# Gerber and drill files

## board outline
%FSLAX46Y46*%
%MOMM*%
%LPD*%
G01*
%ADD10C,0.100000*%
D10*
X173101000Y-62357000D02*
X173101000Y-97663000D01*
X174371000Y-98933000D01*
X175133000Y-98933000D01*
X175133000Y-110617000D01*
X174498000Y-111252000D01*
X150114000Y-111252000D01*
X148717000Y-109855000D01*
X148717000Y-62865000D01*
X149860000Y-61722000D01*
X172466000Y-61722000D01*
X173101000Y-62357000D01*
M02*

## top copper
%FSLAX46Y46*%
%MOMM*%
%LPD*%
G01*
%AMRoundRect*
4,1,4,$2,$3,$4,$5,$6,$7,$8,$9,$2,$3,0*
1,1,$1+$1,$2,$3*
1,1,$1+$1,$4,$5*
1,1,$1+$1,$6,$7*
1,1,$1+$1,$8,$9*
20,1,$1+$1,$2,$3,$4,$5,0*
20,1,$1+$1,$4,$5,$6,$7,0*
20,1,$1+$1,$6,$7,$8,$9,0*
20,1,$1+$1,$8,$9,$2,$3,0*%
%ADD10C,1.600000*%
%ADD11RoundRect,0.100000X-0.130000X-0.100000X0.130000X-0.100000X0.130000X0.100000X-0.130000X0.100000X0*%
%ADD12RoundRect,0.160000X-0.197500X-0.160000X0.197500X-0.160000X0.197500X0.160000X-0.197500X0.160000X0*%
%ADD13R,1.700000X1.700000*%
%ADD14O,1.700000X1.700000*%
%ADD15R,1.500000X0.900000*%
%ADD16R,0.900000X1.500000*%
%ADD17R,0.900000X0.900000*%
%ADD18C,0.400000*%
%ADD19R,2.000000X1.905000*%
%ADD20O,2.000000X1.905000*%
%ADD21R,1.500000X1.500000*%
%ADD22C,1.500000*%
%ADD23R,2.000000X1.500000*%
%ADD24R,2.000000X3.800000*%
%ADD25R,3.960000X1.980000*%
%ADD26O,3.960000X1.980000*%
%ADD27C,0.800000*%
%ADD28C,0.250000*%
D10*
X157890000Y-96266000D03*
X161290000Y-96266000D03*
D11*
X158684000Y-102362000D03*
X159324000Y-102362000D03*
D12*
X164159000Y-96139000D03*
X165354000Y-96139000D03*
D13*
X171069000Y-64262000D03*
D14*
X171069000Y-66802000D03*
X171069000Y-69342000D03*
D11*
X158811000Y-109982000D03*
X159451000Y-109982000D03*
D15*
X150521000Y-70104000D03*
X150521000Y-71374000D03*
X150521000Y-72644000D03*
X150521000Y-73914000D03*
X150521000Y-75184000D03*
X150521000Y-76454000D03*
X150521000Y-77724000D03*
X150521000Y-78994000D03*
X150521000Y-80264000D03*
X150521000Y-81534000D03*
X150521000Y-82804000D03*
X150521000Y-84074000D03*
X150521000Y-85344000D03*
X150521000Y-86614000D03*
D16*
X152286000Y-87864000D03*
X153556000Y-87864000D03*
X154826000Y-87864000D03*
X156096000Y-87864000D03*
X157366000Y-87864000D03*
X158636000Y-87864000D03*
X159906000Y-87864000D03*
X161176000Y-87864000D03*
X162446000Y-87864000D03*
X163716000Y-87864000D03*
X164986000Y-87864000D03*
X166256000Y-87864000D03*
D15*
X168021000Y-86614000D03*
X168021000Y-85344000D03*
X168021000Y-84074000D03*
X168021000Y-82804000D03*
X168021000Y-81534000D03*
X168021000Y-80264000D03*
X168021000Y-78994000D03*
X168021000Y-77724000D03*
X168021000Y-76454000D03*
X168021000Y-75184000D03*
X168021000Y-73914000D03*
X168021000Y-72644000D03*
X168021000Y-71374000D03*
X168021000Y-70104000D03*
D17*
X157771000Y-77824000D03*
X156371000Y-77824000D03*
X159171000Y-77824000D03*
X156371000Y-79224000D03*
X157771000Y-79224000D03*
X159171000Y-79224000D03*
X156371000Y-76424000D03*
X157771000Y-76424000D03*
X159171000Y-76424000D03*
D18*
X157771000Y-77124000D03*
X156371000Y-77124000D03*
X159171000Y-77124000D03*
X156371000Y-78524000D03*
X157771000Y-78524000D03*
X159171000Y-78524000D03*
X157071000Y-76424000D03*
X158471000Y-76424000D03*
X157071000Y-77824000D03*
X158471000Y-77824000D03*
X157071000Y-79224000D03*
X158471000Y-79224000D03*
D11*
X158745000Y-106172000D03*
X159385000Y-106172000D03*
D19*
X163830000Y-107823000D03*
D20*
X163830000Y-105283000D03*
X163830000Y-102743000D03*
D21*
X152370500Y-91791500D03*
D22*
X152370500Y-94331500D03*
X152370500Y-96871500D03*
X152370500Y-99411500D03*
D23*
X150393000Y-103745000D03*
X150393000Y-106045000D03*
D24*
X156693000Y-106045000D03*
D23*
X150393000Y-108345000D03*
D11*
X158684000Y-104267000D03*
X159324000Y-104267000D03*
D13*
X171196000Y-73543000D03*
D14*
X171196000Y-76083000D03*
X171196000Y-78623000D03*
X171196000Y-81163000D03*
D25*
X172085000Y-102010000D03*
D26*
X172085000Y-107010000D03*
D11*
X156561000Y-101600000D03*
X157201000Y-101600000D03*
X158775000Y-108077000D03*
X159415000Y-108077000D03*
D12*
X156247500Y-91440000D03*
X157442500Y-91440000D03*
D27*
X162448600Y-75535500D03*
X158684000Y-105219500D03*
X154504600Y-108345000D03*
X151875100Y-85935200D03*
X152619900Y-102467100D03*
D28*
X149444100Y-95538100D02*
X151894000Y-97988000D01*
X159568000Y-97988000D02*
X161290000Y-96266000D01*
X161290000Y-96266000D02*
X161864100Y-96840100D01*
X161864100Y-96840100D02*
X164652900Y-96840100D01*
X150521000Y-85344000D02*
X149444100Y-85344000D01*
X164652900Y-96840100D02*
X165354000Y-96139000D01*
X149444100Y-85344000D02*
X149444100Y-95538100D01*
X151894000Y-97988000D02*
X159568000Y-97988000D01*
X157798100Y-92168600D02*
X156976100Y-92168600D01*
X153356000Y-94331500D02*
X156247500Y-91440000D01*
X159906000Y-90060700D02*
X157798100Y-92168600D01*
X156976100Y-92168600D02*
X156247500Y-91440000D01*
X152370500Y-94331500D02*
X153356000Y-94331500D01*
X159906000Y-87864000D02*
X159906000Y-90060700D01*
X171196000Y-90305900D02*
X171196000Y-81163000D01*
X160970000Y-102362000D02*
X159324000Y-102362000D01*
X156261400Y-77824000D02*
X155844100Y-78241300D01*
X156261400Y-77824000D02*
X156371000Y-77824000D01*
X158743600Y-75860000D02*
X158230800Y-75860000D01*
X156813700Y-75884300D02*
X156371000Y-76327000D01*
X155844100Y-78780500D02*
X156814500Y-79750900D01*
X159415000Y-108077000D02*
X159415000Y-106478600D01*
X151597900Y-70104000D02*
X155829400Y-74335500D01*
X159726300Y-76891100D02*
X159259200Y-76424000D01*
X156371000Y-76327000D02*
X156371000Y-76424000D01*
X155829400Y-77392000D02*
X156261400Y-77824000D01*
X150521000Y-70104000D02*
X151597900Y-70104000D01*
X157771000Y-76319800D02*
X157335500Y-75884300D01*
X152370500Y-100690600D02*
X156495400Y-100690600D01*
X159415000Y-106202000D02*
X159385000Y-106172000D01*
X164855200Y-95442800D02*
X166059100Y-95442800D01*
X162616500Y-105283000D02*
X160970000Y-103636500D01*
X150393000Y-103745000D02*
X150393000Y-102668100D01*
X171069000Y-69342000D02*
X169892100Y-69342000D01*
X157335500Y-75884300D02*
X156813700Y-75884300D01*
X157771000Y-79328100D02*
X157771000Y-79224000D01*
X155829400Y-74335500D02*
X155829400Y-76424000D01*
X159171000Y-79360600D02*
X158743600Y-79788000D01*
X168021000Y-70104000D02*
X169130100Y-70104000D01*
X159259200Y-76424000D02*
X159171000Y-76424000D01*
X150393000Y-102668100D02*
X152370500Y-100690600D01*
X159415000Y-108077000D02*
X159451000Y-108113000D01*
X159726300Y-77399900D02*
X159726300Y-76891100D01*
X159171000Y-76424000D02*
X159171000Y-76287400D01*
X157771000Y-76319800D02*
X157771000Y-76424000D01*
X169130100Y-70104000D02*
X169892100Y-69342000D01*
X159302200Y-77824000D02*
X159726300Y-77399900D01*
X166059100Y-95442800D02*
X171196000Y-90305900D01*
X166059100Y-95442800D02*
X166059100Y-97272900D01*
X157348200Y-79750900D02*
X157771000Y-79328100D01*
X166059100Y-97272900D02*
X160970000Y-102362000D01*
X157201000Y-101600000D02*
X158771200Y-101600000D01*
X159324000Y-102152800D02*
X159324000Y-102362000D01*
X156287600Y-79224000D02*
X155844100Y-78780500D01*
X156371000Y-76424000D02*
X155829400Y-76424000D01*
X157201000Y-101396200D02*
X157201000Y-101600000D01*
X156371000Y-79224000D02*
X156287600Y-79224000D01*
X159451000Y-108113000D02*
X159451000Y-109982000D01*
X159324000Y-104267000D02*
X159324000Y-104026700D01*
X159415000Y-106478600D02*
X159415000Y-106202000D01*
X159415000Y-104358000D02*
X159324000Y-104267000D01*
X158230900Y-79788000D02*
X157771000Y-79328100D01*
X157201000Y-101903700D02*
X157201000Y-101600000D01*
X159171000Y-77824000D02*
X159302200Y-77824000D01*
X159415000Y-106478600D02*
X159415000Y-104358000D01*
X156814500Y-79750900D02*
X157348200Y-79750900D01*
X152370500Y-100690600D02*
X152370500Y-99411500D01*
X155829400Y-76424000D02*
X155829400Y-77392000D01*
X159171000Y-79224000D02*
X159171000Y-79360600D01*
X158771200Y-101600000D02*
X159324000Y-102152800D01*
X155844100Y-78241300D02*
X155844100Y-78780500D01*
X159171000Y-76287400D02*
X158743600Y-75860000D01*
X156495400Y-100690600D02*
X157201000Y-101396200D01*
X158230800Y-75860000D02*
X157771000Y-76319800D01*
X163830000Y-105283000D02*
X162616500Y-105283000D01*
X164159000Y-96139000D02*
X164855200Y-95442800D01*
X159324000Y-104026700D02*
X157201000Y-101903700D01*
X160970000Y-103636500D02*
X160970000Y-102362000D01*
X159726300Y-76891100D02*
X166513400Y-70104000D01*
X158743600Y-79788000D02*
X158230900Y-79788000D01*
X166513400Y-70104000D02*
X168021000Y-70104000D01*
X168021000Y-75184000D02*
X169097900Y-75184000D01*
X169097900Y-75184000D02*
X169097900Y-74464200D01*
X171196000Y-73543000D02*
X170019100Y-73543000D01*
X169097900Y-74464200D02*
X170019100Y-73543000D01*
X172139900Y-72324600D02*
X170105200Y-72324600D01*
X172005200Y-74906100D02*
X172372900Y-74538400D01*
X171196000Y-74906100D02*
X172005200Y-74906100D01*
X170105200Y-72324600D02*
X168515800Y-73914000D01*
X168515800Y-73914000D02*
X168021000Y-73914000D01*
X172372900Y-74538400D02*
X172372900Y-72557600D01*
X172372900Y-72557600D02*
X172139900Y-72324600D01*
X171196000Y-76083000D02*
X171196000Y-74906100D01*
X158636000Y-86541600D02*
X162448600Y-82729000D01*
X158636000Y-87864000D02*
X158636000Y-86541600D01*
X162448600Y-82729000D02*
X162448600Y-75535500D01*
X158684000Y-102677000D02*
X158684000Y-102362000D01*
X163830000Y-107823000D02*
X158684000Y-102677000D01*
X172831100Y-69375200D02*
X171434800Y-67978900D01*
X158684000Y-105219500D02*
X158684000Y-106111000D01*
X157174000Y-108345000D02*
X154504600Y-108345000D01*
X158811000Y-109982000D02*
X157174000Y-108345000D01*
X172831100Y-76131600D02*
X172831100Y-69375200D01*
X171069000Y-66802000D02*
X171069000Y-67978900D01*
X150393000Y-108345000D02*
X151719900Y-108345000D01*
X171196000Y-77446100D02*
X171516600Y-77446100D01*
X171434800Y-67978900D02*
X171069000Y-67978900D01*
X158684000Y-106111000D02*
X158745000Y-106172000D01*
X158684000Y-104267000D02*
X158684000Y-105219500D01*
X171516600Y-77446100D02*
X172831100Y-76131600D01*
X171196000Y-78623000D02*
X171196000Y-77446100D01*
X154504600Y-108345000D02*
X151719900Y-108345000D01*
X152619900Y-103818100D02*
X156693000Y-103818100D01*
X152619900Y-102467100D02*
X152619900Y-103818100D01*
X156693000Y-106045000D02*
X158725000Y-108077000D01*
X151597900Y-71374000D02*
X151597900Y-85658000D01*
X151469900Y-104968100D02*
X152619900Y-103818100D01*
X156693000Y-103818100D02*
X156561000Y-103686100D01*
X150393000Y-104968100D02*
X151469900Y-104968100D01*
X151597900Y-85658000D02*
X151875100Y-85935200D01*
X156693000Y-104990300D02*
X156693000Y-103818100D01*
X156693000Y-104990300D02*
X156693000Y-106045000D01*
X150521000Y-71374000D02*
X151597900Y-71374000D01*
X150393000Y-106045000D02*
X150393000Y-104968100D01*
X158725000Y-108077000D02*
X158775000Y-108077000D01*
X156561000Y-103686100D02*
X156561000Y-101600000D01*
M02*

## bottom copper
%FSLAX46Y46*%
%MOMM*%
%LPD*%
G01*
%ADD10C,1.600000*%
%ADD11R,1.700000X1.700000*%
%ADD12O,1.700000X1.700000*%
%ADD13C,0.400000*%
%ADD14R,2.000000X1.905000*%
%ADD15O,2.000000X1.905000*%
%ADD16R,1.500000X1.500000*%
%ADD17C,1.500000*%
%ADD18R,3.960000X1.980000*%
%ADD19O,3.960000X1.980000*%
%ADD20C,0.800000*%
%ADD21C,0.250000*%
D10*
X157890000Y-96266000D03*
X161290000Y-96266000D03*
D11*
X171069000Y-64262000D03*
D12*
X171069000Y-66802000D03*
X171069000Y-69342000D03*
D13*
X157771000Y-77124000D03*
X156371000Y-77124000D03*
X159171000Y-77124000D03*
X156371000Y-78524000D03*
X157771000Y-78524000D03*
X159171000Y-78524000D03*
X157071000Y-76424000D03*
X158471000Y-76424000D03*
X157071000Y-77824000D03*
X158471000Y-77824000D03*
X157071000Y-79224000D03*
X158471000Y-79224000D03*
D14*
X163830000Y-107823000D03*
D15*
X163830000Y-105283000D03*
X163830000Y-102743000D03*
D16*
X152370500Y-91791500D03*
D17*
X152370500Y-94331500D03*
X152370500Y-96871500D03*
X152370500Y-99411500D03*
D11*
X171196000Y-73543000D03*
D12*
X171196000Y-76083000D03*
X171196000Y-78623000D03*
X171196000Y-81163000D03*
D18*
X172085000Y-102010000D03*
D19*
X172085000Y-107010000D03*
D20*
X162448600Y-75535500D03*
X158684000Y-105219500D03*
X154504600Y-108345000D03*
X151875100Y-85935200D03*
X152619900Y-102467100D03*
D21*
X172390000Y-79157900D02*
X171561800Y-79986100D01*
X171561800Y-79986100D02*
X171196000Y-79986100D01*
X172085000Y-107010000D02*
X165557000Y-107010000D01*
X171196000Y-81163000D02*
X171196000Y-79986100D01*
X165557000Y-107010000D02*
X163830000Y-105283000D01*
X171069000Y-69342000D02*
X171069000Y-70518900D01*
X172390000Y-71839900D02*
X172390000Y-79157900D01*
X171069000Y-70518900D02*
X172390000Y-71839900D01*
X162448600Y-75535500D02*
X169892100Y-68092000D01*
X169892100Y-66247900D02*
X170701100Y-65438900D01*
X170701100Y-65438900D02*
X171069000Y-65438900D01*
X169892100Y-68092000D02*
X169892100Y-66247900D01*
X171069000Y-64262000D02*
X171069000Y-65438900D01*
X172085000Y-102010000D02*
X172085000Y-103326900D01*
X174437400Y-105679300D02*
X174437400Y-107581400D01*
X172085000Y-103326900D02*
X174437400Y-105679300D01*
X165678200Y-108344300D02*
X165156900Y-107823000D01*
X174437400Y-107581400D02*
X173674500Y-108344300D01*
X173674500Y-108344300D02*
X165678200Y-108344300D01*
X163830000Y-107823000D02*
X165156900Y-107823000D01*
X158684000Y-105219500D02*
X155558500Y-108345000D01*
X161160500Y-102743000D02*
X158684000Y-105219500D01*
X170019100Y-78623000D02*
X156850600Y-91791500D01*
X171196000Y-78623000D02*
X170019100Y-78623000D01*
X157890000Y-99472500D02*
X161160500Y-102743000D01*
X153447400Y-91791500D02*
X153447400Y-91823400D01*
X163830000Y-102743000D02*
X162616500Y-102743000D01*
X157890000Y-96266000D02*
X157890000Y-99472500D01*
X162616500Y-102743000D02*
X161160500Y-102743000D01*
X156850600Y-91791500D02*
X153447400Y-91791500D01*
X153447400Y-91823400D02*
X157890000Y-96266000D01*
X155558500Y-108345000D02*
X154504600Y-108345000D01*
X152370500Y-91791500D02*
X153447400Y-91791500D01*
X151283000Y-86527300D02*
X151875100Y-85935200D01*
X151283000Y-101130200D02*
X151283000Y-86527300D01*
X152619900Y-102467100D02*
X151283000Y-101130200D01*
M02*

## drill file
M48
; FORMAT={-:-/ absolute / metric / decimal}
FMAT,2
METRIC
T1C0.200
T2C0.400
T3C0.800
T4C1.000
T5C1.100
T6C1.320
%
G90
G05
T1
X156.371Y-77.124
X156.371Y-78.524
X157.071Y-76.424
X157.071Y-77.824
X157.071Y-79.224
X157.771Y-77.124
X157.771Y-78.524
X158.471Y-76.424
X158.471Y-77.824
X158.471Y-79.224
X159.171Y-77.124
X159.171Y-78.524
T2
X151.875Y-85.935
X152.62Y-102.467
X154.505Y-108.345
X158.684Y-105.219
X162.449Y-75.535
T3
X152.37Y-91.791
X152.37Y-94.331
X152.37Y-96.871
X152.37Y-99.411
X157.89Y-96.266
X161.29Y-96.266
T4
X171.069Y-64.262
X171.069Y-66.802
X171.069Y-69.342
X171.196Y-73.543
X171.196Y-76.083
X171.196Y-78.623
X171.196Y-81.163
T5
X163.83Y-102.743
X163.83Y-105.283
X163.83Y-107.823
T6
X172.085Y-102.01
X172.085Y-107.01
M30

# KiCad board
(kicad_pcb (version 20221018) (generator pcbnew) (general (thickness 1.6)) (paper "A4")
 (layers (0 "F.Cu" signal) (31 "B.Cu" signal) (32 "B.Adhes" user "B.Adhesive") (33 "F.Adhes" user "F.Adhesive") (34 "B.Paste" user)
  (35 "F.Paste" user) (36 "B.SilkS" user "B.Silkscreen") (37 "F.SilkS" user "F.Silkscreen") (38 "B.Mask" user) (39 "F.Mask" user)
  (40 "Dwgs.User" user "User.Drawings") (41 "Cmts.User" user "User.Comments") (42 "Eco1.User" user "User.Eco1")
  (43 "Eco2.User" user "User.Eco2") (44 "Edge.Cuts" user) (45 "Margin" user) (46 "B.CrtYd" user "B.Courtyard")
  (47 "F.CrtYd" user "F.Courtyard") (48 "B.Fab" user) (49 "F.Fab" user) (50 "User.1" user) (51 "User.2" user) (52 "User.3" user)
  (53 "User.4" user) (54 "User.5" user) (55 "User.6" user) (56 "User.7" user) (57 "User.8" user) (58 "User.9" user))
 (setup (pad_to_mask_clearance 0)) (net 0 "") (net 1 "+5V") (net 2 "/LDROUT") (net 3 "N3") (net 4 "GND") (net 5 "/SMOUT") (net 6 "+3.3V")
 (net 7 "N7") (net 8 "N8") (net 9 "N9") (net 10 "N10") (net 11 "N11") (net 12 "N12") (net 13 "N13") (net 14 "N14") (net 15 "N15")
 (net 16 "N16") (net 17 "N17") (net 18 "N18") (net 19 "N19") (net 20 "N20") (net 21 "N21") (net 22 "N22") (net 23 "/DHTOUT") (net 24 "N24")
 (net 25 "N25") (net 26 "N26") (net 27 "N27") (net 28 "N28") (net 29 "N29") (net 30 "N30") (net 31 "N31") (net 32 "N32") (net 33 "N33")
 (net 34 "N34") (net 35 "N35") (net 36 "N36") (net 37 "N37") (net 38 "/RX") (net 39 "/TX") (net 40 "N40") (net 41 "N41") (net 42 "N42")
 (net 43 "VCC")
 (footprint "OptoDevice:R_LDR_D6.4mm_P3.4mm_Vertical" (layer "F.Cu") (at 157.89 96.266)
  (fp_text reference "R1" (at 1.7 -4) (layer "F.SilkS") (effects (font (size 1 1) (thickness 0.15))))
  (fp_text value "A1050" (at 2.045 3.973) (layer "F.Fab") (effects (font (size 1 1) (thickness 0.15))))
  (pad "1" thru_hole circle (at 0 0) (size 1.6 1.6) (drill 0.8) (layers "*.Cu" "*.Mask") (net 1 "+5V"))
  (pad "2" thru_hole circle (at 3.4 0) (size 1.6 1.6) (drill 0.8) (layers "*.Cu" "*.Mask") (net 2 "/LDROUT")))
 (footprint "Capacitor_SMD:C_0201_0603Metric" (layer "F.Cu") (at 159.004 102.362)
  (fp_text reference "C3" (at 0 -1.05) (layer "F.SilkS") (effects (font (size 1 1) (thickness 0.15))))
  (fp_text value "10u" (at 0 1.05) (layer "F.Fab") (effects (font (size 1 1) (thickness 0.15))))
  (pad "" smd roundrect (at -0.345 0) (size 0.318 0.36) (layers "F.Paste") (roundrect_rratio 0.25))
  (pad "" smd roundrect (at 0.345 0) (size 0.318 0.36) (layers "F.Paste") (roundrect_rratio 0.25))
  (pad "1" smd roundrect (at -0.32 0) (size 0.46 0.4) (layers "F.Cu" "F.Mask") (roundrect_rratio 0.25) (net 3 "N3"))
  (pad "2" smd roundrect (at 0.32 0) (size 0.46 0.4) (layers "F.Cu" "F.Mask") (roundrect_rratio 0.25) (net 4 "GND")))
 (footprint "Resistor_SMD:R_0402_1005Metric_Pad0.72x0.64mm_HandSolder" (layer "F.Cu") (at 164.7565 96.139)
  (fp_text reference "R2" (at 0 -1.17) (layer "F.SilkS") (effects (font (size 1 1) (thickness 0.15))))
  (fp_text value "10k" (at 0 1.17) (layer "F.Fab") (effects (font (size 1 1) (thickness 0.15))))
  (pad "1" smd roundrect (at -0.5975 0) (size 0.715 0.64) (layers "F.Cu" "F.Paste" "F.Mask") (roundrect_rratio 0.25) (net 4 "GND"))
  (pad "2" smd roundrect (at 0.5975 0) (size 0.715 0.64) (layers "F.Cu" "F.Paste" "F.Mask") (roundrect_rratio 0.25) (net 2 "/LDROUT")))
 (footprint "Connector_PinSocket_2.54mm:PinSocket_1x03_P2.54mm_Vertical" (layer "F.Cu") (at 171.069 64.262)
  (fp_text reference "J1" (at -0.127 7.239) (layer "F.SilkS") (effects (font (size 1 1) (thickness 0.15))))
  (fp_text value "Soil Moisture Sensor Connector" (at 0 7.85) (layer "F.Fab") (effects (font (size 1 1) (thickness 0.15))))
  (pad "1" thru_hole rect (at 0 0) (size 1.7 1.7) (drill 1) (layers "*.Cu" "*.Mask") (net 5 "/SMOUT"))
  (pad "2" thru_hole oval (at 0 2.54) (size 1.7 1.7) (drill 1) (layers "*.Cu" "*.Mask") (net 1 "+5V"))
  (pad "3" thru_hole oval (at 0 5.08) (size 1.7 1.7) (drill 1) (layers "*.Cu" "*.Mask") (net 4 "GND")))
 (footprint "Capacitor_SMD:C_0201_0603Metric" (layer "F.Cu") (at 159.131 109.982)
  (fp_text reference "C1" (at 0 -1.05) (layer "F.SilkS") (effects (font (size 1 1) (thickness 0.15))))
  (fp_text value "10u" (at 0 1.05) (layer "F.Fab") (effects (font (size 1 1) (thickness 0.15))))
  (pad "" smd roundrect (at -0.345 0) (size 0.318 0.36) (layers "F.Paste") (roundrect_rratio 0.25))
  (pad "" smd roundrect (at 0.345 0) (size 0.318 0.36) (layers "F.Paste") (roundrect_rratio 0.25))
  (pad "1" smd roundrect (at -0.32 0) (size 0.46 0.4) (layers "F.Cu" "F.Mask") (roundrect_rratio 0.25) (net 1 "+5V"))
  (pad "2" smd roundrect (at 0.32 0) (size 0.46 0.4) (layers "F.Cu" "F.Mask") (roundrect_rratio 0.25) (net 4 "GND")))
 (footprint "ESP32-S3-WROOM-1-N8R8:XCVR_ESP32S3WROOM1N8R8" (layer "F.Cu") (at 159.271 75.364)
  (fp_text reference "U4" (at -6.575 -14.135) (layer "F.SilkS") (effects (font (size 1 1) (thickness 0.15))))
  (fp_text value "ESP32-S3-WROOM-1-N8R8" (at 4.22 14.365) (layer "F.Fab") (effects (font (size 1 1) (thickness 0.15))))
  (pad "1" smd rect (at -8.75 -5.26) (size 1.5 0.9) (layers "F.Cu" "F.Paste" "F.Mask") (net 4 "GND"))
  (pad "2" smd rect (at -8.75 -3.99) (size 1.5 0.9) (layers "F.Cu" "F.Paste" "F.Mask") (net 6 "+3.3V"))
  (pad "3" smd rect (at -8.75 -2.72) (size 1.5 0.9) (layers "F.Cu" "F.Paste" "F.Mask") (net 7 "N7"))
  (pad "4" smd rect (at -8.75 -1.45) (size 1.5 0.9) (layers "F.Cu" "F.Paste" "F.Mask") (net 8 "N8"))
  (pad "5" smd rect (at -8.75 -0.18) (size 1.5 0.9) (layers "F.Cu" "F.Paste" "F.Mask") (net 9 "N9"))
  (pad "6" smd rect (at -8.75 1.09) (size 1.5 0.9) (layers "F.Cu" "F.Paste" "F.Mask") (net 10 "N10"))
  (pad "7" smd rect (at -8.75 2.36) (size 1.5 0.9) (layers "F.Cu" "F.Paste" "F.Mask") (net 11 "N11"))
  (pad "8" smd rect (at -8.75 3.63) (size 1.5 0.9) (layers "F.Cu" "F.Paste" "F.Mask") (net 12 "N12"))
  (pad "9" smd rect (at -8.75 4.9) (size 1.5 0.9) (layers "F.Cu" "F.Paste" "F.Mask") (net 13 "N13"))
  (pad "10" smd rect (at -8.75 6.17) (size 1.5 0.9) (layers "F.Cu" "F.Paste" "F.Mask") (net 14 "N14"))
  (pad "11" smd rect (at -8.75 7.44) (size 1.5 0.9) (layers "F.Cu" "F.Paste" "F.Mask") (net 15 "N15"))
  (pad "12" smd rect (at -8.75 8.71) (size 1.5 0.9) (layers "F.Cu" "F.Paste" "F.Mask") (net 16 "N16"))
  (pad "13" smd rect (at -8.75 9.98) (size 1.5 0.9) (layers "F.Cu" "F.Paste" "F.Mask") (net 2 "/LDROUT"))
  (pad "14" smd rect (at -8.75 11.25) (size 1.5 0.9) (layers "F.Cu" "F.Paste" "F.Mask") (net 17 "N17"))
  (pad "15" smd rect (at -6.985 12.5) (size 0.9 1.5) (layers "F.Cu" "F.Paste" "F.Mask") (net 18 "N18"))
  (pad "16" smd rect (at -5.715 12.5) (size 0.9 1.5) (layers "F.Cu" "F.Paste" "F.Mask") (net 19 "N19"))
  (pad "17" smd rect (at -4.445 12.5) (size 0.9 1.5) (layers "F.Cu" "F.Paste" "F.Mask") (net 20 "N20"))
  (pad "18" smd rect (at -3.175 12.5) (size 0.9 1.5) (layers "F.Cu" "F.Paste" "F.Mask") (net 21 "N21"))
  (pad "19" smd rect (at -1.905 12.5) (size 0.9 1.5) (layers "F.Cu" "F.Paste" "F.Mask") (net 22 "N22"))
  (pad "20" smd rect (at -0.635 12.5) (size 0.9 1.5) (layers "F.Cu" "F.Paste" "F.Mask") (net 5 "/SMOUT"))
  (pad "21" smd rect (at 0.635 12.5) (size 0.9 1.5) (layers "F.Cu" "F.Paste" "F.Mask") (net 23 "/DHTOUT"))
  (pad "22" smd rect (at 1.905 12.5) (size 0.9 1.5) (layers "F.Cu" "F.Paste" "F.Mask") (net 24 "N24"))
  (pad "23" smd rect (at 3.175 12.5) (size 0.9 1.5) (layers "F.Cu" "F.Paste" "F.Mask") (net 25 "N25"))
  (pad "24" smd rect (at 4.445 12.5) (size 0.9 1.5) (layers "F.Cu" "F.Paste" "F.Mask") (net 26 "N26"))
  (pad "25" smd rect (at 5.715 12.5) (size 0.9 1.5) (layers "F.Cu" "F.Paste" "F.Mask") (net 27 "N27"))
  (pad "26" smd rect (at 6.985 12.5) (size 0.9 1.5) (layers "F.Cu" "F.Paste" "F.Mask") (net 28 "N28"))
  (pad "27" smd rect (at 8.75 11.25) (size 1.5 0.9) (layers "F.Cu" "F.Paste" "F.Mask") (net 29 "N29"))
  (pad "28" smd rect (at 8.75 9.98) (size 1.5 0.9) (layers "F.Cu" "F.Paste" "F.Mask") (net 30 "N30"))
  (pad "29" smd rect (at 8.75 8.71) (size 1.5 0.9) (layers "F.Cu" "F.Paste" "F.Mask") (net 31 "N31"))
  (pad "30" smd rect (at 8.75 7.44) (size 1.5 0.9) (layers "F.Cu" "F.Paste" "F.Mask") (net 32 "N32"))
  (pad "31" smd rect (at 8.75 6.17) (size 1.5 0.9) (layers "F.Cu" "F.Paste" "F.Mask") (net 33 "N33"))
  (pad "32" smd rect (at 8.75 4.9) (size 1.5 0.9) (layers "F.Cu" "F.Paste" "F.Mask") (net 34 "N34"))
  (pad "33" smd rect (at 8.75 3.63) (size 1.5 0.9) (layers "F.Cu" "F.Paste" "F.Mask") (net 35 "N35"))
  (pad "34" smd rect (at 8.75 2.36) (size 1.5 0.9) (layers "F.Cu" "F.Paste" "F.Mask") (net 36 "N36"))
  (pad "35" smd rect (at 8.75 1.09) (size 1.5 0.9) (layers "F.Cu" "F.Paste" "F.Mask") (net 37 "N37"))
  (pad "36" smd rect (at 8.75 -0.18) (size 1.5 0.9) (layers "F.Cu" "F.Paste" "F.Mask") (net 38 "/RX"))
  (pad "37" smd rect (at 8.75 -1.45) (size 1.5 0.9) (layers "F.Cu" "F.Paste" "F.Mask") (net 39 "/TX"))
  (pad "38" smd rect (at 8.75 -2.72) (size 1.5 0.9) (layers "F.Cu" "F.Paste" "F.Mask") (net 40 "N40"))
  (pad "39" smd rect (at 8.75 -3.99) (size 1.5 0.9) (layers "F.Cu" "F.Paste" "F.Mask") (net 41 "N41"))
  (pad "40" smd rect (at 8.75 -5.26) (size 1.5 0.9) (layers "F.Cu" "F.Paste" "F.Mask") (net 4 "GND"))
  (pad "41_1" smd rect (at -1.5 2.46) (size 0.9 0.9) (layers "F.Cu" "F.Paste" "F.Mask") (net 4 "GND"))
  (pad "41_2" smd rect (at -2.9 2.46) (size 0.9 0.9) (layers "F.Cu" "F.Paste" "F.Mask") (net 4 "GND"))
  (pad "41_3" smd rect (at -0.1 2.46) (size 0.9 0.9) (layers "F.Cu" "F.Paste" "F.Mask") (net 4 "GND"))
  (pad "41_4" smd rect (at -2.9 3.86) (size 0.9 0.9) (layers "F.Cu" "F.Paste" "F.Mask") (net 4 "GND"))
  (pad "41_5" smd rect (at -1.5 3.86) (size 0.9 0.9) (layers "F.Cu" "F.Paste" "F.Mask") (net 4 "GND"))
  (pad "41_6" smd rect (at -0.1 3.86) (size 0.9 0.9) (layers "F.Cu" "F.Paste" "F.Mask") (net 4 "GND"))
  (pad "41_7" smd rect (at -2.9 1.06) (size 0.9 0.9) (layers "F.Cu" "F.Paste" "F.Mask") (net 4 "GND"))
  (pad "41_8" smd rect (at -1.5 1.06) (size 0.9 0.9) (layers "F.Cu" "F.Paste" "F.Mask") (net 4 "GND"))
  (pad "41_9" smd rect (at -0.1 1.06) (size 0.9 0.9) (layers "F.Cu" "F.Paste" "F.Mask") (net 4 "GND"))
  (pad "41_10" thru_hole circle (at -1.5 1.76) (size 0.4 0.4) (drill 0.2) (layers "*.Cu"))
  (pad "41_11" thru_hole circle (at -2.9 1.76) (size 0.4 0.4) (drill 0.2) (layers "*.Cu"))
  (pad "41_12" thru_hole circle (at -0.1 1.76) (size 0.4 0.4) (drill 0.2) (layers "*.Cu"))
  (pad "41_13" thru_hole circle (at -2.9 3.16) (size 0.4 0.4) (drill 0.2) (layers "*.Cu"))
  (pad "41_14" thru_hole circle (at -1.5 3.16) (size 0.4 0.4) (drill 0.2) (layers "*.Cu"))
  (pad "41_15" thru_hole circle (at -0.1 3.16) (size 0.4 0.4) (drill 0.2) (layers "*.Cu"))
  (pad "41_16" thru_hole circle (at -2.2 1.06) (size 0.4 0.4) (drill 0.2) (layers "*.Cu"))
  (pad "41_17" thru_hole circle (at -0.8 1.06) (size 0.4 0.4) (drill 0.2) (layers "*.Cu"))
  (pad "41_18" thru_hole circle (at -2.2 2.46) (size 0.4 0.4) (drill 0.2) (layers "*.Cu"))
  (pad "41_19" thru_hole circle (at -0.8 2.46) (size 0.4 0.4) (drill 0.2) (layers "*.Cu"))
  (pad "41_20" thru_hole circle (at -2.2 3.86) (size 0.4 0.4) (drill 0.2) (layers "*.Cu"))
  (pad "41_21" thru_hole circle (at -0.8 3.86) (size 0.4 0.4) (drill 0.2) (layers "*.Cu"))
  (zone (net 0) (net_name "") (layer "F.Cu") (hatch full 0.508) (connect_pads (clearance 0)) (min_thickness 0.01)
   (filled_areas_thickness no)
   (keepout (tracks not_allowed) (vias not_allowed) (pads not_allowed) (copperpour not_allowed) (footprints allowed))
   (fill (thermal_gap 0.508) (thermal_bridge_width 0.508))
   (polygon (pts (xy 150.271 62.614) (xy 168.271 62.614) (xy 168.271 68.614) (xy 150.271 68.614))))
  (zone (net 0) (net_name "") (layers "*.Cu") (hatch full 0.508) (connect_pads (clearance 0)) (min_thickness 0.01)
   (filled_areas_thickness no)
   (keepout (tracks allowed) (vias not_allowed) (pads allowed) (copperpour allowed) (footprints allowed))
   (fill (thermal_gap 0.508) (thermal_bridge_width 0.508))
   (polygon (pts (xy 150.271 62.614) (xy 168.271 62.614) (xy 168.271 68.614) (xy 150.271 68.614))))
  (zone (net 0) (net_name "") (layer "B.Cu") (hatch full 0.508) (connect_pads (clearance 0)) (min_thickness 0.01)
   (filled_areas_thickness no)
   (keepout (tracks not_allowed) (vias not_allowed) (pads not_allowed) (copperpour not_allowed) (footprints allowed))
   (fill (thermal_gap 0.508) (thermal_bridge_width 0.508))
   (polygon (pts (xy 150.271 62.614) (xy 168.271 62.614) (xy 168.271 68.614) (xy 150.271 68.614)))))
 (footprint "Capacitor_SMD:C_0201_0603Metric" (layer "F.Cu") (at 159.065 106.172)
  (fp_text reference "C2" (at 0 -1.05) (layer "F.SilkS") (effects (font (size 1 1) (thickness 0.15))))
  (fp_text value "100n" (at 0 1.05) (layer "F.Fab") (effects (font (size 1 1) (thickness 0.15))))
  (pad "" smd roundrect (at -0.345 0) (size 0.318 0.36) (layers "F.Paste") (roundrect_rratio 0.25))
  (pad "" smd roundrect (at 0.345 0) (size 0.318 0.36) (layers "F.Paste") (roundrect_rratio 0.25))
  (pad "1" smd roundrect (at -0.32 0) (size 0.46 0.4) (layers "F.Cu" "F.Mask") (roundrect_rratio 0.25) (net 1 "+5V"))
  (pad "2" smd roundrect (at 0.32 0) (size 0.46 0.4) (layers "F.Cu" "F.Mask") (roundrect_rratio 0.25) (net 4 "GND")))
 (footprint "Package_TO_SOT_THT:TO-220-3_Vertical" (layer "F.Cu") (at 163.83 107.823 90)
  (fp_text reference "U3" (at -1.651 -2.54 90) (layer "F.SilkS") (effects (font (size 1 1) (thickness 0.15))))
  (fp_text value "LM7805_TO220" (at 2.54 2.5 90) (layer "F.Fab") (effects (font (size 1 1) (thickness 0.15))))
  (pad "1" thru_hole rect (at 0 0 90) (size 1.905 2) (drill 1.1) (layers "*.Cu" "*.Mask") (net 3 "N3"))
  (pad "2" thru_hole oval (at 2.54 0 90) (size 1.905 2) (drill 1.1) (layers "*.Cu" "*.Mask") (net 4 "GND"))
  (pad "3" thru_hole oval (at 5.08 0 90) (size 1.905 2) (drill 1.1) (layers "*.Cu" "*.Mask") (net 1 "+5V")))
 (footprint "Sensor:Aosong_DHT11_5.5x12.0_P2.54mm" (layer "F.Cu") (at 152.3705 91.7915)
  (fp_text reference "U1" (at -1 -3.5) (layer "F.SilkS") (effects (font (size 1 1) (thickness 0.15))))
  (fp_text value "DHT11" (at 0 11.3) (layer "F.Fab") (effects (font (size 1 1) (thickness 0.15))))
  (pad "1" thru_hole rect (at 0 0) (size 1.5 1.5) (drill 0.8) (layers "*.Cu" "*.Mask") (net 1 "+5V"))
  (pad "2" thru_hole circle (at 0 2.54) (size 1.5 1.5) (drill 0.8) (layers "*.Cu" "*.Mask") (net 23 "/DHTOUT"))
  (pad "3" thru_hole circle (at 0 5.08) (size 1.5 1.5) (drill 0.8) (layers "*.Cu" "*.Mask") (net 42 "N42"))
  (pad "4" thru_hole circle (at 0 7.62) (size 1.5 1.5) (drill 0.8) (layers "*.Cu" "*.Mask") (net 4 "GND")))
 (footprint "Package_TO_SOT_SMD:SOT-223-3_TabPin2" (layer "F.Cu") (at 153.543 106.045)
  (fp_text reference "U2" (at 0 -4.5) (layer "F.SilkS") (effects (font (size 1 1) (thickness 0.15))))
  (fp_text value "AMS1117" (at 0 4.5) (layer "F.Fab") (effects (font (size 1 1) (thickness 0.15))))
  (pad "1" smd rect (at -3.15 -2.3) (size 2 1.5) (layers "F.Cu" "F.Paste" "F.Mask") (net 4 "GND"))
  (pad "2" smd rect (at -3.15 0) (size 2 1.5) (layers "F.Cu" "F.Paste" "F.Mask") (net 6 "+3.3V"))
  (pad "2" smd rect (at 3.15 0) (size 2 3.8) (layers "F.Cu" "F.Paste" "F.Mask") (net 6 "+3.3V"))
  (pad "3" smd rect (at -3.15 2.3) (size 2 1.5) (layers "F.Cu" "F.Paste" "F.Mask") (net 1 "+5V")))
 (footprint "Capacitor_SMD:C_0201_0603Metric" (layer "F.Cu") (at 159.004 104.267)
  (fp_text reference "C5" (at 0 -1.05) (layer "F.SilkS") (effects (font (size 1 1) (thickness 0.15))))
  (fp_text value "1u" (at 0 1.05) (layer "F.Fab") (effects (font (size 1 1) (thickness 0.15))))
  (pad "" smd roundrect (at -0.345 0) (size 0.318 0.36) (layers "F.Paste") (roundrect_rratio 0.25))
  (pad "" smd roundrect (at 0.345 0) (size 0.318 0.36) (layers "F.Paste") (roundrect_rratio 0.25))
  (pad "1" smd roundrect (at -0.32 0) (size 0.46 0.4) (layers "F.Cu" "F.Mask") (roundrect_rratio 0.25) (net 1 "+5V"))
  (pad "2" smd roundrect (at 0.32 0) (size 0.46 0.4) (layers "F.Cu" "F.Mask") (roundrect_rratio 0.25) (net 4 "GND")))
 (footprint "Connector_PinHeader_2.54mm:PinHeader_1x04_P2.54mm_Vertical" (layer "F.Cu") (at 171.196 73.543)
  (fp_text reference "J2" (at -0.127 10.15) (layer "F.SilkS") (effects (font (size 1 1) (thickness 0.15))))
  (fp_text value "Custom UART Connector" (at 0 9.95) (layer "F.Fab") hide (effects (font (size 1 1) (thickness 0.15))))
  (pad "1" thru_hole rect (at 0 0) (size 1.7 1.7) (drill 1) (layers "*.Cu" "*.Mask") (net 38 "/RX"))
  (pad "2" thru_hole oval (at 0 2.54) (size 1.7 1.7) (drill 1) (layers "*.Cu" "*.Mask") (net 39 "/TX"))
  (pad "3" thru_hole oval (at 0 5.08) (size 1.7 1.7) (drill 1) (layers "*.Cu" "*.Mask") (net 1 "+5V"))
  (pad "4" thru_hole oval (at 0 7.62) (size 1.7 1.7) (drill 1) (layers "*.Cu" "*.Mask") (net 4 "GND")))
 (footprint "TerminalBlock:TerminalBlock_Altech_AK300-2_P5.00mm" (layer "F.Cu") (at 172.085 102.01 -90)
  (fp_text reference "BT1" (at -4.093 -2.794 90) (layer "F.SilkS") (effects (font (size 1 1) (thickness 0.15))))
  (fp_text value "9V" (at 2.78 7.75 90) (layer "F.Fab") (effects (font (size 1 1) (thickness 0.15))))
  (pad "1" thru_hole rect (at 0 0 270) (size 1.98 3.96) (drill 1.32) (layers "*.Cu" "*.Mask") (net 3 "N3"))
  (pad "2" thru_hole oval (at 5 0 270) (size 1.98 3.96) (drill 1.32) (layers "*.Cu" "*.Mask") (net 4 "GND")))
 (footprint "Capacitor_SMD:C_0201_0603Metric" (layer "F.Cu") (at 156.881 101.6)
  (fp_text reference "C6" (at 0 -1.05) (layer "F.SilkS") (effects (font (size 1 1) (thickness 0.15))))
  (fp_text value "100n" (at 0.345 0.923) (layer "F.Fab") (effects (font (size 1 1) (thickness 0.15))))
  (pad "" smd roundrect (at -0.345 0) (size 0.318 0.36) (layers "F.Paste") (roundrect_rratio 0.25))
  (pad "" smd roundrect (at 0.345 0) (size 0.318 0.36) (layers "F.Paste") (roundrect_rratio 0.25))
  (pad "1" smd roundrect (at -0.32 0) (size 0.46 0.4) (layers "F.Cu" "F.Mask") (roundrect_rratio 0.25) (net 6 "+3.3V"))
  (pad "2" smd roundrect (at 0.32 0) (size 0.46 0.4) (layers "F.Cu" "F.Mask") (roundrect_rratio 0.25) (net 4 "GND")))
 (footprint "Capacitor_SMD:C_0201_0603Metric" (layer "F.Cu") (at 159.095 108.077)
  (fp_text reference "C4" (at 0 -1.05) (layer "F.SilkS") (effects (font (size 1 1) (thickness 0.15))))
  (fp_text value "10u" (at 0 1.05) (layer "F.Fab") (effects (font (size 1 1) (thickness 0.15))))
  (pad "" smd roundrect (at -0.345 0) (size 0.318 0.36) (layers "F.Paste") (roundrect_rratio 0.25))
  (pad "" smd roundrect (at 0.345 0) (size 0.318 0.36) (layers "F.Paste") (roundrect_rratio 0.25))
  (pad "1" smd roundrect (at -0.32 0) (size 0.46 0.4) (layers "F.Cu" "F.Mask") (roundrect_rratio 0.25) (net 6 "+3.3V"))
  (pad "2" smd roundrect (at 0.32 0) (size 0.46 0.4) (layers "F.Cu" "F.Mask") (roundrect_rratio 0.25) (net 4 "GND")))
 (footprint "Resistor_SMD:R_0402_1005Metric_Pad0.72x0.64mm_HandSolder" (layer "F.Cu") (at 156.845 91.44)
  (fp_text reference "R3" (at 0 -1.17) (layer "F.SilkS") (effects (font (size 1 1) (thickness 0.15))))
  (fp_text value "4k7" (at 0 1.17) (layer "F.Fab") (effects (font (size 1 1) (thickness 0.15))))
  (pad "1" smd roundrect (at -0.5975 0) (size 0.715 0.64) (layers "F.Cu" "F.Paste" "F.Mask") (roundrect_rratio 0.25) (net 23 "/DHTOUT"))
  (pad "2" smd roundrect (at 0.5975 0) (size 0.715 0.64) (layers "F.Cu" "F.Paste" "F.Mask") (roundrect_rratio 0.25) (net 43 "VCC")))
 (gr_poly
  (pts (xy 173.101 62.357) (xy 173.101 97.663) (xy 174.371 98.933) (xy 175.133 98.933) (xy 175.133 110.617) (xy 174.498 111.252)
   (xy 150.114 111.252) (xy 148.717 109.855) (xy 148.717 62.865) (xy 149.86 61.722) (xy 172.466 61.722))
  (stroke (width 0.1) (type solid)) (fill none) (layer "Edge.Cuts"))
 (segment (start 149.4441 95.5381) (end 151.894 97.988) (width 0.25) (layer "F.Cu") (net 2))
 (segment (start 159.568 97.988) (end 161.29 96.266) (width 0.25) (layer "F.Cu") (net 2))
 (segment (start 161.29 96.266) (end 161.8641 96.8401) (width 0.25) (layer "F.Cu") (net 2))
 (segment (start 161.8641 96.8401) (end 164.6529 96.8401) (width 0.25) (layer "F.Cu") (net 2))
 (segment (start 150.521 85.344) (end 149.4441 85.344) (width 0.25) (layer "F.Cu") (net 2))
 (segment (start 164.6529 96.8401) (end 165.354 96.139) (width 0.25) (layer "F.Cu") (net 2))
 (segment (start 149.4441 85.344) (end 149.4441 95.5381) (width 0.25) (layer "F.Cu") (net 2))
 (segment (start 151.894 97.988) (end 159.568 97.988) (width 0.25) (layer "F.Cu") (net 2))
 (segment (start 157.7981 92.1686) (end 156.9761 92.1686) (width 0.25) (layer "F.Cu") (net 23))
 (segment (start 153.356 94.3315) (end 156.2475 91.44) (width 0.25) (layer "F.Cu") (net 23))
 (segment (start 159.906 90.0607) (end 157.7981 92.1686) (width 0.25) (layer "F.Cu") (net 23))
 (segment (start 156.9761 92.1686) (end 156.2475 91.44) (width 0.25) (layer "F.Cu") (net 23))
 (segment (start 152.3705 94.3315) (end 153.356 94.3315) (width 0.25) (layer "F.Cu") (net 23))
 (segment (start 159.906 87.864) (end 159.906 90.0607) (width 0.25) (layer "F.Cu") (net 23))
 (segment (start 171.196 90.3059) (end 171.196 81.163) (width 0.25) (layer "F.Cu") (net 4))
 (segment (start 160.97 102.362) (end 159.324 102.362) (width 0.25) (layer "F.Cu") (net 4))
 (segment (start 156.2614 77.824) (end 155.8441 78.2413) (width 0.25) (layer "F.Cu") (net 4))
 (segment (start 156.2614 77.824) (end 156.371 77.824) (width 0.25) (layer "F.Cu") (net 4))
 (segment (start 158.7436 75.86) (end 158.2308 75.86) (width 0.25) (layer "F.Cu") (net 4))
 (segment (start 156.8137 75.8843) (end 156.371 76.327) (width 0.25) (layer "F.Cu") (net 4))
 (segment (start 155.8441 78.7805) (end 156.8145 79.7509) (width 0.25) (layer "F.Cu") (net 4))
 (segment (start 159.415 108.077) (end 159.415 106.4786) (width 0.25) (layer "F.Cu") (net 4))
 (segment (start 151.5979 70.104) (end 155.8294 74.3355) (width 0.25) (layer "F.Cu") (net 4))
 (segment (start 159.7263 76.8911) (end 159.2592 76.424) (width 0.25) (layer "F.Cu") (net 4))
 (segment (start 156.371 76.327) (end 156.371 76.424) (width 0.25) (layer "F.Cu") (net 4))
 (segment (start 155.8294 77.392) (end 156.2614 77.824) (width 0.25) (layer "F.Cu") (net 4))
 (segment (start 150.521 70.104) (end 151.5979 70.104) (width 0.25) (layer "F.Cu") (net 4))
 (segment (start 157.771 76.3198) (end 157.3355 75.8843) (width 0.25) (layer "F.Cu") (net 4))
 (segment (start 152.3705 100.6906) (end 156.4954 100.6906) (width 0.25) (layer "F.Cu") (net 4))
 (segment (start 159.415 106.202) (end 159.385 106.172) (width 0.25) (layer "F.Cu") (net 4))
 (segment (start 164.8552 95.4428) (end 166.0591 95.4428) (width 0.25) (layer "F.Cu") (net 4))
 (segment (start 162.6165 105.283) (end 160.97 103.6365) (width 0.25) (layer "F.Cu") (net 4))
 (segment (start 150.393 103.745) (end 150.393 102.6681) (width 0.25) (layer "F.Cu") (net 4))
 (segment (start 171.069 69.342) (end 169.8921 69.342) (width 0.25) (layer "F.Cu") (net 4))
 (segment (start 157.3355 75.8843) (end 156.8137 75.8843) (width 0.25) (layer "F.Cu") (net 4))
 (segment (start 157.771 79.3281) (end 157.771 79.224) (width 0.25) (layer "F.Cu") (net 4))
 (segment (start 155.8294 74.3355) (end 155.8294 76.424) (width 0.25) (layer "F.Cu") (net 4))
 (segment (start 159.171 79.3606) (end 158.7436 79.788) (width 0.25) (layer "F.Cu") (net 4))
 (segment (start 168.021 70.104) (end 169.1301 70.104) (width 0.25) (layer "F.Cu") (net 4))
 (segment (start 159.2592 76.424) (end 159.171 76.424) (width 0.25) (layer "F.Cu") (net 4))
 (segment (start 150.393 102.6681) (end 152.3705 100.6906) (width 0.25) (layer "F.Cu") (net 4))
 (segment (start 159.415 108.077) (end 159.451 108.113) (width 0.25) (layer "F.Cu") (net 4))
 (segment (start 159.7263 77.3999) (end 159.7263 76.8911) (width 0.25) (layer "F.Cu") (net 4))
 (segment (start 159.171 76.424) (end 159.171 76.2874) (width 0.25) (layer "F.Cu") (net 4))
 (segment (start 157.771 76.3198) (end 157.771 76.424) (width 0.25) (layer "F.Cu") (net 4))
 (segment (start 169.1301 70.104) (end 169.8921 69.342) (width 0.25) (layer "F.Cu") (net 4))
 (segment (start 159.3022 77.824) (end 159.7263 77.3999) (width 0.25) (layer "F.Cu") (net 4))
 (segment (start 166.0591 95.4428) (end 171.196 90.3059) (width 0.25) (layer "F.Cu") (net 4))
 (segment (start 166.0591 95.4428) (end 166.0591 97.2729) (width 0.25) (layer "F.Cu") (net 4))
 (segment (start 157.3482 79.7509) (end 157.771 79.3281) (width 0.25) (layer "F.Cu") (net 4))
 (segment (start 166.0591 97.2729) (end 160.97 102.362) (width 0.25) (layer "F.Cu") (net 4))
 (segment (start 157.201 101.6) (end 158.7712 101.6) (width 0.25) (layer "F.Cu") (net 4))
 (segment (start 159.324 102.1528) (end 159.324 102.362) (width 0.25) (layer "F.Cu") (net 4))
 (segment (start 156.2876 79.224) (end 155.8441 78.7805) (width 0.25) (layer "F.Cu") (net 4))
 (segment (start 156.371 76.424) (end 155.8294 76.424) (width 0.25) (layer "F.Cu") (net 4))
 (segment (start 157.201 101.3962) (end 157.201 101.6) (width 0.25) (layer "F.Cu") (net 4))
 (segment (start 156.371 79.224) (end 156.2876 79.224) (width 0.25) (layer "F.Cu") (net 4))
 (segment (start 159.451 108.113) (end 159.451 109.982) (width 0.25) (layer "F.Cu") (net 4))
 (segment (start 159.324 104.267) (end 159.324 104.0267) (width 0.25) (layer "F.Cu") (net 4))
 (segment (start 159.415 106.4786) (end 159.415 106.202) (width 0.25) (layer "F.Cu") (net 4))
 (segment (start 159.415 104.358) (end 159.324 104.267) (width 0.25) (layer "F.Cu") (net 4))
 (segment (start 158.2309 79.788) (end 157.771 79.3281) (width 0.25) (layer "F.Cu") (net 4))
 (segment (start 157.201 101.9037) (end 157.201 101.6) (width 0.25) (layer "F.Cu") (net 4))
 (segment (start 159.171 77.824) (end 159.3022 77.824) (width 0.25) (layer "F.Cu") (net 4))
 (segment (start 159.415 106.4786) (end 159.415 104.358) (width 0.25) (layer "F.Cu") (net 4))
 (segment (start 156.8145 79.7509) (end 157.3482 79.7509) (width 0.25) (layer "F.Cu") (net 4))
 (segment (start 152.3705 100.6906) (end 152.3705 99.4115) (width 0.25) (layer "F.Cu") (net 4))
 (segment (start 155.8294 76.424) (end 155.8294 77.392) (width 0.25) (layer "F.Cu") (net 4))
 (segment (start 159.171 79.224) (end 159.171 79.3606) (width 0.25) (layer "F.Cu") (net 4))
 (segment (start 158.7712 101.6) (end 159.324 102.1528) (width 0.25) (layer "F.Cu") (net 4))
 (segment (start 155.8441 78.2413) (end 155.8441 78.7805) (width 0.25) (layer "F.Cu") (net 4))
 (segment (start 159.171 76.2874) (end 158.7436 75.86) (width 0.25) (layer "F.Cu") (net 4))
 (segment (start 156.4954 100.6906) (end 157.201 101.3962) (width 0.25) (layer "F.Cu") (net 4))
 (segment (start 158.2308 75.86) (end 157.771 76.3198) (width 0.25) (layer "F.Cu") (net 4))
 (segment (start 163.83 105.283) (end 162.6165 105.283) (width 0.25) (layer "F.Cu") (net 4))
 (segment (start 164.159 96.139) (end 164.8552 95.4428) (width 0.25) (layer "F.Cu") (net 4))
 (segment (start 159.324 104.0267) (end 157.201 101.9037) (width 0.25) (layer "F.Cu") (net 4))
 (segment (start 160.97 103.6365) (end 160.97 102.362) (width 0.25) (layer "F.Cu") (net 4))
 (segment (start 159.7263 76.8911) (end 166.5134 70.104) (width 0.25) (layer "F.Cu") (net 4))
 (segment (start 158.7436 79.788) (end 158.2309 79.788) (width 0.25) (layer "F.Cu") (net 4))
 (segment (start 166.5134 70.104) (end 168.021 70.104) (width 0.25) (layer "F.Cu") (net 4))
 (segment (start 172.39 79.1579) (end 171.5618 79.9861) (width 0.25) (layer "B.Cu") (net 4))
 (segment (start 171.5618 79.9861) (end 171.196 79.9861) (width 0.25) (layer "B.Cu") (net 4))
 (segment (start 172.085 107.01) (end 165.557 107.01) (width 0.25) (layer "B.Cu") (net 4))
 (segment (start 171.196 81.163) (end 171.196 79.9861) (width 0.25) (layer "B.Cu") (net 4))
 (segment (start 165.557 107.01) (end 163.83 105.283) (width 0.25) (layer "B.Cu") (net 4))
 (segment (start 171.069 69.342) (end 171.069 70.5189) (width 0.25) (layer "B.Cu") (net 4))
 (segment (start 172.39 71.8399) (end 172.39 79.1579) (width 0.25) (layer "B.Cu") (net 4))
 (segment (start 171.069 70.5189) (end 172.39 71.8399) (width 0.25) (layer "B.Cu") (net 4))
 (segment (start 168.021 75.184) (end 169.0979 75.184) (width 0.25) (layer "F.Cu") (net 38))
 (segment (start 169.0979 75.184) (end 169.0979 74.4642) (width 0.25) (layer "F.Cu") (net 38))
 (segment (start 171.196 73.543) (end 170.0191 73.543) (width 0.25) (layer "F.Cu") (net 38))
 (segment (start 169.0979 74.4642) (end 170.0191 73.543) (width 0.25) (layer "F.Cu") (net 38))
 (segment (start 172.1399 72.3246) (end 170.1052 72.3246) (width 0.25) (layer "F.Cu") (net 39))
 (segment (start 172.0052 74.9061) (end 172.3729 74.5384) (width 0.25) (layer "F.Cu") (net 39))
 (segment (start 171.196 74.9061) (end 172.0052 74.9061) (width 0.25) (layer "F.Cu") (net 39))
 (segment (start 170.1052 72.3246) (end 168.5158 73.914) (width 0.25) (layer "F.Cu") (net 39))
 (segment (start 168.5158 73.914) (end 168.021 73.914) (width 0.25) (layer "F.Cu") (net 39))
 (segment (start 172.3729 74.5384) (end 172.3729 72.5576) (width 0.25) (layer "F.Cu") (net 39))
 (segment (start 172.3729 72.5576) (end 172.1399 72.3246) (width 0.25) (layer "F.Cu") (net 39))
 (segment (start 171.196 76.083) (end 171.196 74.9061) (width 0.25) (layer "F.Cu") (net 39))
 (segment (start 158.636 86.5416) (end 162.4486 82.729) (width 0.25) (layer "F.Cu") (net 5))
 (segment (start 158.636 87.864) (end 158.636 86.5416) (width 0.25) (layer "F.Cu") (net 5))
 (segment (start 162.4486 82.729) (end 162.4486 75.5355) (width 0.25) (layer "F.Cu") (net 5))
 (via (at 162.4486 75.5355) (size 0.8) (drill 0.4) (layers "F.Cu" "B.Cu") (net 5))
 (segment (start 162.4486 75.5355) (end 169.8921 68.092) (width 0.25) (layer "B.Cu") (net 5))
 (segment (start 169.8921 66.2479) (end 170.7011 65.4389) (width 0.25) (layer "B.Cu") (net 5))
 (segment (start 170.7011 65.4389) (end 171.069 65.4389) (width 0.25) (layer "B.Cu") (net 5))
 (segment (start 169.8921 68.092) (end 169.8921 66.2479) (width 0.25) (layer "B.Cu") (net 5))
 (segment (start 171.069 64.262) (end 171.069 65.4389) (width 0.25) (layer "B.Cu") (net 5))
 (segment (start 158.684 102.677) (end 158.684 102.362) (width 0.25) (layer "F.Cu") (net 3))
 (segment (start 163.83 107.823) (end 158.684 102.677) (width 0.25) (layer "F.Cu") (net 3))
 (segment (start 172.085 102.01) (end 172.085 103.3269) (width 0.25) (layer "B.Cu") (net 3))
 (segment (start 174.4374 105.6793) (end 174.4374 107.5814) (width 0.25) (layer "B.Cu") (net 3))
 (segment (start 172.085 103.3269) (end 174.4374 105.6793) (width 0.25) (layer "B.Cu") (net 3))
 (segment (start 165.6782 108.3443) (end 165.1569 107.823) (width 0.25) (layer "B.Cu") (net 3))
 (segment (start 174.4374 107.5814) (end 173.6745 108.3443) (width 0.25) (layer "B.Cu") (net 3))
 (segment (start 173.6745 108.3443) (end 165.6782 108.3443) (width 0.25) (layer "B.Cu") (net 3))
 (segment (start 163.83 107.823) (end 165.1569 107.823) (width 0.25) (layer "B.Cu") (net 3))
 (segment (start 172.8311 69.3752) (end 171.4348 67.9789) (width 0.25) (layer "F.Cu") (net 1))
 (segment (start 158.684 105.2195) (end 158.684 106.111) (width 0.25) (layer "F.Cu") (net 1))
 (segment (start 157.174 108.345) (end 154.5046 108.345) (width 0.25) (layer "F.Cu") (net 1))
 (segment (start 158.811 109.982) (end 157.174 108.345) (width 0.25) (layer "F.Cu") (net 1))
 (segment (start 172.8311 76.1316) (end 172.8311 69.3752) (width 0.25) (layer "F.Cu") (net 1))
 (segment (start 171.069 66.802) (end 171.069 67.9789) (width 0.25) (layer "F.Cu") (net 1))
 (segment (start 150.393 108.345) (end 151.7199 108.345) (width 0.25) (layer "F.Cu") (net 1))
 (segment (start 171.196 77.4461) (end 171.5166 77.4461) (width 0.25) (layer "F.Cu") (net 1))
 (segment (start 171.4348 67.9789) (end 171.069 67.9789) (width 0.25) (layer "F.Cu") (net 1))
 (segment (start 158.684 106.111) (end 158.745 106.172) (width 0.25) (layer "F.Cu") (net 1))
 (segment (start 158.684 104.267) (end 158.684 105.2195) (width 0.25) (layer "F.Cu") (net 1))
 (segment (start 171.5166 77.4461) (end 172.8311 76.1316) (width 0.25) (layer "F.Cu") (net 1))
 (segment (start 171.196 78.623) (end 171.196 77.4461) (width 0.25) (layer "F.Cu") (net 1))
 (segment (start 154.5046 108.345) (end 151.7199 108.345) (width 0.25) (layer "F.Cu") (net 1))
 (via (at 158.684 105.2195) (size 0.8) (drill 0.4) (layers "F.Cu" "B.Cu") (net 1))
 (via (at 154.5046 108.345) (size 0.8) (drill 0.4) (layers "F.Cu" "B.Cu") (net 1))
 (segment (start 158.684 105.2195) (end 155.5585 108.345) (width 0.25) (layer "B.Cu") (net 1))
 (segment (start 161.1605 102.743) (end 158.684 105.2195) (width 0.25) (layer "B.Cu") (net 1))
 (segment (start 170.0191 78.623) (end 156.8506 91.7915) (width 0.25) (layer "B.Cu") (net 1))
 (segment (start 171.196 78.623) (end 170.0191 78.623) (width 0.25) (layer "B.Cu") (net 1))
 (segment (start 157.89 99.4725) (end 161.1605 102.743) (width 0.25) (layer "B.Cu") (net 1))
 (segment (start 153.4474 91.7915) (end 153.4474 91.8234) (width 0.25) (layer "B.Cu") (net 1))
 (segment (start 163.83 102.743) (end 162.6165 102.743) (width 0.25) (layer "B.Cu") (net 1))
 (segment (start 157.89 96.266) (end 157.89 99.4725) (width 0.25) (layer "B.Cu") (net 1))
 (segment (start 162.6165 102.743) (end 161.1605 102.743) (width 0.25) (layer "B.Cu") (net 1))
 (segment (start 156.8506 91.7915) (end 153.4474 91.7915) (width 0.25) (layer "B.Cu") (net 1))
 (segment (start 153.4474 91.8234) (end 157.89 96.266) (width 0.25) (layer "B.Cu") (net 1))
 (segment (start 155.5585 108.345) (end 154.5046 108.345) (width 0.25) (layer "B.Cu") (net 1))
 (segment (start 152.3705 91.7915) (end 153.4474 91.7915) (width 0.25) (layer "B.Cu") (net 1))
 (segment (start 152.6199 103.8181) (end 156.693 103.8181) (width 0.25) (layer "F.Cu") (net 6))
 (segment (start 152.6199 102.4671) (end 152.6199 103.8181) (width 0.25) (layer "F.Cu") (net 6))
 (segment (start 156.693 106.045) (end 158.725 108.077) (width 0.25) (layer "F.Cu") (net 6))
 (segment (start 151.5979 71.374) (end 151.5979 85.658) (width 0.25) (layer "F.Cu") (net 6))
 (segment (start 151.4699 104.9681) (end 152.6199 103.8181) (width 0.25) (layer "F.Cu") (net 6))
 (segment (start 156.693 103.8181) (end 156.561 103.6861) (width 0.25) (layer "F.Cu") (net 6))
 (segment (start 150.393 104.9681) (end 151.4699 104.9681) (width 0.25) (layer "F.Cu") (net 6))
 (segment (start 151.5979 85.658) (end 151.8751 85.9352) (width 0.25) (layer "F.Cu") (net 6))
 (segment (start 156.693 104.9903) (end 156.693 103.8181) (width 0.25) (layer "F.Cu") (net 6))
 (segment (start 156.693 104.9903) (end 156.693 106.045) (width 0.25) (layer "F.Cu") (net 6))
 (segment (start 150.521 71.374) (end 151.5979 71.374) (width 0.25) (layer "F.Cu") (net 6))
 (segment (start 150.393 106.045) (end 150.393 104.9681) (width 0.25) (layer "F.Cu") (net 6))
 (segment (start 158.725 108.077) (end 158.775 108.077) (width 0.25) (layer "F.Cu") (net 6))
 (segment (start 156.561 103.6861) (end 156.561 101.6) (width 0.25) (layer "F.Cu") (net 6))
 (via (at 151.8751 85.9352) (size 0.8) (drill 0.4) (layers "F.Cu" "B.Cu") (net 6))
 (via (at 152.6199 102.4671) (size 0.8) (drill 0.4) (layers "F.Cu" "B.Cu") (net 6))
 (segment (start 151.283 86.5273) (end 151.8751 85.9352) (width 0.25) (layer "B.Cu") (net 6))
 (segment (start 151.283 101.1302) (end 151.283 86.5273) (width 0.25) (layer "B.Cu") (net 6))
 (segment (start 152.6199 102.4671) (end 151.283 101.1302) (width 0.25) (layer "B.Cu") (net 6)))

